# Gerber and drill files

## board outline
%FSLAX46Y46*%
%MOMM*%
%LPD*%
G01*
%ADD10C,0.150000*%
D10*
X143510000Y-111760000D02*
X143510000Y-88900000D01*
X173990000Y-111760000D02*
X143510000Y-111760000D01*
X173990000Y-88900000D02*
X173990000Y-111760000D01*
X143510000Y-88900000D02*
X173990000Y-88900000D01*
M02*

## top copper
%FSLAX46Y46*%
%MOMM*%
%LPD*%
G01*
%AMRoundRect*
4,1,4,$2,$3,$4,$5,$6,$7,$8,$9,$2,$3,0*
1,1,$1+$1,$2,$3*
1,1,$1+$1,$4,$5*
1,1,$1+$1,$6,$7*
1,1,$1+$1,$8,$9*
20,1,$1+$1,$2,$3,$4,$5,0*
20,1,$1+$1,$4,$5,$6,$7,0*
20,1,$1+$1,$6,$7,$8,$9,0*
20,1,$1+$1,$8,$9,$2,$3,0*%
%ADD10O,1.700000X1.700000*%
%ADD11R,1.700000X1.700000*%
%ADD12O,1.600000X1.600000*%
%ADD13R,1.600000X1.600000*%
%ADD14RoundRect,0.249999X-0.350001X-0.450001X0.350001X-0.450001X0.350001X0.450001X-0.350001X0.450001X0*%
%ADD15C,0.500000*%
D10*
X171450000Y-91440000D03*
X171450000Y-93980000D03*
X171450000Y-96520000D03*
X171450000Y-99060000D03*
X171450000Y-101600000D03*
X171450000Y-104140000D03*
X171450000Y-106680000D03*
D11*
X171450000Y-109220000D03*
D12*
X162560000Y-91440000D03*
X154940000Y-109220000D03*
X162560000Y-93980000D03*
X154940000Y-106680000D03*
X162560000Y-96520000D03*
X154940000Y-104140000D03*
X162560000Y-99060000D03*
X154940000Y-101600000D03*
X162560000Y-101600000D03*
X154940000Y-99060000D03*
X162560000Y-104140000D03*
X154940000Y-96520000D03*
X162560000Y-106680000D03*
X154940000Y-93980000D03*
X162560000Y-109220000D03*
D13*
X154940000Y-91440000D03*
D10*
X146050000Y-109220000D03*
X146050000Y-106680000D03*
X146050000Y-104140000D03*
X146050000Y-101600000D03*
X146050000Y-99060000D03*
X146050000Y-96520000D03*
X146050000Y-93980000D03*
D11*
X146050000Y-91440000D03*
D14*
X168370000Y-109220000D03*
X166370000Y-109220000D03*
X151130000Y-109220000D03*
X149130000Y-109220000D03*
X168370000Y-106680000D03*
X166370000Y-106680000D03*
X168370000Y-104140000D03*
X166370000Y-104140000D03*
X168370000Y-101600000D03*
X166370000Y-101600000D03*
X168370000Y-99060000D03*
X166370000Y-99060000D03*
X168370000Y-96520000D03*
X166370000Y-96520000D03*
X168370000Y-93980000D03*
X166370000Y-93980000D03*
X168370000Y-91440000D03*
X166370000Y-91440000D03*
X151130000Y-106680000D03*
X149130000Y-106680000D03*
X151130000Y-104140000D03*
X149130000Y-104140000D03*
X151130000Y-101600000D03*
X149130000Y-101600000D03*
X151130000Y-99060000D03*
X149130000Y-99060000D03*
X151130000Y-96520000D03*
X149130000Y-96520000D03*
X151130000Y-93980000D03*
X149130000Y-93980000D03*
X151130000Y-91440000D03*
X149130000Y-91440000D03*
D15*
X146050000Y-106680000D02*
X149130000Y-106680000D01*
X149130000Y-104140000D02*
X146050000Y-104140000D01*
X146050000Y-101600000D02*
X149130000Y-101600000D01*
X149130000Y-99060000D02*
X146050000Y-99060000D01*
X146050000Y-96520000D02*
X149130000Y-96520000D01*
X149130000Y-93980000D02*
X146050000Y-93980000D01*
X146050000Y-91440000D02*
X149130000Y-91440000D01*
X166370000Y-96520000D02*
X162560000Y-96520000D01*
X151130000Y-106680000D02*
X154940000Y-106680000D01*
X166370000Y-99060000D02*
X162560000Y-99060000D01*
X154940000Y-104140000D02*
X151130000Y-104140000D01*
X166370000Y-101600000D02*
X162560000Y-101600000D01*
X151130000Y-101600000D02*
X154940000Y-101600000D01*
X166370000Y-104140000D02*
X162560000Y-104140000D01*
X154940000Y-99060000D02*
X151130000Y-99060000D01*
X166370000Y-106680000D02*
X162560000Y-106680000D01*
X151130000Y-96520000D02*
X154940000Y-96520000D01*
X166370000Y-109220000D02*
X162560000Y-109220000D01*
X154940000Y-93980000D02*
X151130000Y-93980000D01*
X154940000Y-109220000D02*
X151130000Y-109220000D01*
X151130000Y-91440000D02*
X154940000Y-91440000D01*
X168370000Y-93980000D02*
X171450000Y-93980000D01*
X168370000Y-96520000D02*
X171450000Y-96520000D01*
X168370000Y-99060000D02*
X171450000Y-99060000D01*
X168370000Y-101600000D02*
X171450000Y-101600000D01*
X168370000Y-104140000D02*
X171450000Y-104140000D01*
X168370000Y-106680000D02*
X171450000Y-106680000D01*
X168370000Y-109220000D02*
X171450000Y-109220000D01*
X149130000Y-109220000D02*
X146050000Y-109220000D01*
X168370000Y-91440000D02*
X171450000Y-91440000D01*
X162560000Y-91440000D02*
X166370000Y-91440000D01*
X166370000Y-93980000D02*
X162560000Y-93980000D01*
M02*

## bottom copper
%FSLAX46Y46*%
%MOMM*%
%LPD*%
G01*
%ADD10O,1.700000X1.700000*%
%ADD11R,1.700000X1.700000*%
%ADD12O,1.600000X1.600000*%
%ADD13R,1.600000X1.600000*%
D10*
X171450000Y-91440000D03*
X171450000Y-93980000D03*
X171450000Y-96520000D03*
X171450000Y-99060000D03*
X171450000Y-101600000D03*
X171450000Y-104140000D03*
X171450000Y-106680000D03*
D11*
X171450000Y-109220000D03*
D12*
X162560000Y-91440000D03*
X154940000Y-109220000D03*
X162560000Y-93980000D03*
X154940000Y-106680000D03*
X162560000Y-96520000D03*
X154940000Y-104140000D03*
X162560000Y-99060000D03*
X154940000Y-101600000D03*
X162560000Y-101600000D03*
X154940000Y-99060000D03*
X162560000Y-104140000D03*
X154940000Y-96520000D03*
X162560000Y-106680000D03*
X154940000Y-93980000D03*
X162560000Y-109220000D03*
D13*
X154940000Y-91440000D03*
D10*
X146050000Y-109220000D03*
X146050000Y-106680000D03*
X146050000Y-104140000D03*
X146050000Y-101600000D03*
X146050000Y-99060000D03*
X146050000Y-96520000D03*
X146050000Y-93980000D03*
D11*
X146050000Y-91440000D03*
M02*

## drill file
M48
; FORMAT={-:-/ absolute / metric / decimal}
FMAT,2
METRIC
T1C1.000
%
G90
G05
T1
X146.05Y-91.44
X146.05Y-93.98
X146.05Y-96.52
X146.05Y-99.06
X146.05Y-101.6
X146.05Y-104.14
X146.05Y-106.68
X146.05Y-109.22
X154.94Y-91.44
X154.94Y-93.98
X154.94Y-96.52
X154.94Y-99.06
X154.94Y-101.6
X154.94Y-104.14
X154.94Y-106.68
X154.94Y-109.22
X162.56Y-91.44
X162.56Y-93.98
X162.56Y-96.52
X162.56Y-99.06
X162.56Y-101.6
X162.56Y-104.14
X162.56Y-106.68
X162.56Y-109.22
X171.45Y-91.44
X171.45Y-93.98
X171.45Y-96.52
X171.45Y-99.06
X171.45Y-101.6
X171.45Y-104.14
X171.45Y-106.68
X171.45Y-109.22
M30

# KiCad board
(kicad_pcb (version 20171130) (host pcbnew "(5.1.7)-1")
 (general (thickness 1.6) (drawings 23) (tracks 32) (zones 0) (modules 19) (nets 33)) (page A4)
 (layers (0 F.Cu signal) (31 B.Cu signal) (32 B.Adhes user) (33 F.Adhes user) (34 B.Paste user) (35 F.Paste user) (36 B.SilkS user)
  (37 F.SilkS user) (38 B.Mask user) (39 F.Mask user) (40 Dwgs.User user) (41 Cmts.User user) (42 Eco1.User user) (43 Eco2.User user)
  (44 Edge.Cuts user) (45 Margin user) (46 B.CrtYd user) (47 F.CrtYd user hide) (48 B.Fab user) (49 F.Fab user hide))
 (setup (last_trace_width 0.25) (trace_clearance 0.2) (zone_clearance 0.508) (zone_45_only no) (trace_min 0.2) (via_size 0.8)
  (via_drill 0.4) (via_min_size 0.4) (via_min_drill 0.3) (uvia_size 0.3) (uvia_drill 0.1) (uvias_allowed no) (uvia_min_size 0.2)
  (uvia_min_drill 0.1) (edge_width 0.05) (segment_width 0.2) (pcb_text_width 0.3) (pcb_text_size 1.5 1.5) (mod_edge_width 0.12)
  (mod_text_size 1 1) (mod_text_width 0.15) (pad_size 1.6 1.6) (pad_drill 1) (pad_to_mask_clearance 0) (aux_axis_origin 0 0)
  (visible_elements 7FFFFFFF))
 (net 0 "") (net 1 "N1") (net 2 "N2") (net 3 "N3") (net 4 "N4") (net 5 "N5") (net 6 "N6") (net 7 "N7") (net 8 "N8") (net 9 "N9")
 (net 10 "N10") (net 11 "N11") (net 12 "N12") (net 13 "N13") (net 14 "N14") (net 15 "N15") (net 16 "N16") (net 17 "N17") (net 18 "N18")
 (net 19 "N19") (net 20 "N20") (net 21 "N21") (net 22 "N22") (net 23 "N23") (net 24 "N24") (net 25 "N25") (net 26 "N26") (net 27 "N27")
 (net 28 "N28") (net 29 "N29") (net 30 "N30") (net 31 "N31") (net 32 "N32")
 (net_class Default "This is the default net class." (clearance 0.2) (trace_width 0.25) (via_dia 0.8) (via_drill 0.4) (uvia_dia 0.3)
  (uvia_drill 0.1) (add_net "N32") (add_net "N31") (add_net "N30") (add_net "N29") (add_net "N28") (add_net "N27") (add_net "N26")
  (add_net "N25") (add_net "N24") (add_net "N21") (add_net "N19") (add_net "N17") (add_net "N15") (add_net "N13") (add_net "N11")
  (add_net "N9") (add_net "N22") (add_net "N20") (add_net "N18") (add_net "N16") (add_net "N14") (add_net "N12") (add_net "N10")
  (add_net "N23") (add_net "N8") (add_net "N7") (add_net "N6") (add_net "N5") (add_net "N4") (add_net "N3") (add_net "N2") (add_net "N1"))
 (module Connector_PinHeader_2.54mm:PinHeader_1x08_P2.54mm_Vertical (layer F.Cu) (at 171.45 109.22 180)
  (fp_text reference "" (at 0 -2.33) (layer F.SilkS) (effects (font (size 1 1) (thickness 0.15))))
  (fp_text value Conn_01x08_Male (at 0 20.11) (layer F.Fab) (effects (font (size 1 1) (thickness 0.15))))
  (pad 8 thru_hole oval (at 0 17.78 180) (size 1.7 1.7) (drill 1) (layers *.Cu *.Mask) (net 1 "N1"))
  (pad 7 thru_hole oval (at 0 15.24 180) (size 1.7 1.7) (drill 1) (layers *.Cu *.Mask) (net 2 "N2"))
  (pad 6 thru_hole oval (at 0 12.7 180) (size 1.7 1.7) (drill 1) (layers *.Cu *.Mask) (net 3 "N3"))
  (pad 5 thru_hole oval (at 0 10.16 180) (size 1.7 1.7) (drill 1) (layers *.Cu *.Mask) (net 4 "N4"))
  (pad 4 thru_hole oval (at 0 7.62 180) (size 1.7 1.7) (drill 1) (layers *.Cu *.Mask) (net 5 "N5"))
  (pad 3 thru_hole oval (at 0 5.08 180) (size 1.7 1.7) (drill 1) (layers *.Cu *.Mask) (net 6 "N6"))
  (pad 2 thru_hole oval (at 0 2.54 180) (size 1.7 1.7) (drill 1) (layers *.Cu *.Mask) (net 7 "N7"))
  (pad 1 thru_hole rect (at 0 0 180) (size 1.7 1.7) (drill 1) (layers *.Cu *.Mask) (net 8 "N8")))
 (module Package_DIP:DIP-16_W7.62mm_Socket (layer F.Cu) (at 154.94 91.44)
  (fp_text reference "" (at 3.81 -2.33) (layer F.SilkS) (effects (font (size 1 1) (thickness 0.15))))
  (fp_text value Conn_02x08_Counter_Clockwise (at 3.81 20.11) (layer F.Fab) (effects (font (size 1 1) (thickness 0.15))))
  (pad 16 thru_hole oval (at 7.62 0) (size 1.6 1.6) (drill 1) (layers *.Cu *.Mask) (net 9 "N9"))
  (pad 8 thru_hole oval (at 0 17.78) (size 1.6 1.6) (drill 1) (layers *.Cu *.Mask) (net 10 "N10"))
  (pad 15 thru_hole oval (at 7.62 2.54) (size 1.6 1.6) (drill 1) (layers *.Cu *.Mask) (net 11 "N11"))
  (pad 7 thru_hole oval (at 0 15.24) (size 1.6 1.6) (drill 1) (layers *.Cu *.Mask) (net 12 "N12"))
  (pad 14 thru_hole oval (at 7.62 5.08) (size 1.6 1.6) (drill 1) (layers *.Cu *.Mask) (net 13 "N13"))
  (pad 6 thru_hole oval (at 0 12.7) (size 1.6 1.6) (drill 1) (layers *.Cu *.Mask) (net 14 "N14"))
  (pad 13 thru_hole oval (at 7.62 7.62) (size 1.6 1.6) (drill 1) (layers *.Cu *.Mask) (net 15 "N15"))
  (pad 5 thru_hole oval (at 0 10.16) (size 1.6 1.6) (drill 1) (layers *.Cu *.Mask) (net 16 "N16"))
  (pad 12 thru_hole oval (at 7.62 10.16) (size 1.6 1.6) (drill 1) (layers *.Cu *.Mask) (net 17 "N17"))
  (pad 4 thru_hole oval (at 0 7.62) (size 1.6 1.6) (drill 1) (layers *.Cu *.Mask) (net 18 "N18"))
  (pad 11 thru_hole oval (at 7.62 12.7) (size 1.6 1.6) (drill 1) (layers *.Cu *.Mask) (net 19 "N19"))
  (pad 3 thru_hole oval (at 0 5.08) (size 1.6 1.6) (drill 1) (layers *.Cu *.Mask) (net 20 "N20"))
  (pad 10 thru_hole oval (at 7.62 15.24) (size 1.6 1.6) (drill 1) (layers *.Cu *.Mask) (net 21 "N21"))
  (pad 2 thru_hole oval (at 0 2.54) (size 1.6 1.6) (drill 1) (layers *.Cu *.Mask) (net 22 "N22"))
  (pad 9 thru_hole oval (at 7.62 17.78) (size 1.6 1.6) (drill 1) (layers *.Cu *.Mask) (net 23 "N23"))
  (pad 1 thru_hole rect (at 0 0) (size 1.6 1.6) (drill 1) (layers *.Cu *.Mask) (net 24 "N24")))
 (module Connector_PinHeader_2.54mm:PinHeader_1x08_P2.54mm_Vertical (layer F.Cu) (at 146.05 91.44)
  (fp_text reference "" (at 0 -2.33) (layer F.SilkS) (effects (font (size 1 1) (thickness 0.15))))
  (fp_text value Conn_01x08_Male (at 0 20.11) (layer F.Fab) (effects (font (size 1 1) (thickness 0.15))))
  (pad 8 thru_hole oval (at 0 17.78) (size 1.7 1.7) (drill 1) (layers *.Cu *.Mask) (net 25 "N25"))
  (pad 7 thru_hole oval (at 0 15.24) (size 1.7 1.7) (drill 1) (layers *.Cu *.Mask) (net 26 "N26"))
  (pad 6 thru_hole oval (at 0 12.7) (size 1.7 1.7) (drill 1) (layers *.Cu *.Mask) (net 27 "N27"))
  (pad 5 thru_hole oval (at 0 10.16) (size 1.7 1.7) (drill 1) (layers *.Cu *.Mask) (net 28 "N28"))
  (pad 4 thru_hole oval (at 0 7.62) (size 1.7 1.7) (drill 1) (layers *.Cu *.Mask) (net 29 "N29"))
  (pad 3 thru_hole oval (at 0 5.08) (size 1.7 1.7) (drill 1) (layers *.Cu *.Mask) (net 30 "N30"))
  (pad 2 thru_hole oval (at 0 2.54) (size 1.7 1.7) (drill 1) (layers *.Cu *.Mask) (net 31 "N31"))
  (pad 1 thru_hole rect (at 0 0) (size 1.7 1.7) (drill 1) (layers *.Cu *.Mask) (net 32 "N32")))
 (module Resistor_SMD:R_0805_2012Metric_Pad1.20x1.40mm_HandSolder (layer F.Cu) (at 167.37 109.22)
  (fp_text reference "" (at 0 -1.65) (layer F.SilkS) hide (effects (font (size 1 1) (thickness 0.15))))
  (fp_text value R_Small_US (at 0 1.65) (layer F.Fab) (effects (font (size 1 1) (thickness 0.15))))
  (pad 2 smd roundrect (at 1 0) (size 1.2 1.4) (layers F.Cu F.Paste F.Mask) (roundrect_rratio 0.2083325) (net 8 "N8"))
  (pad 1 smd roundrect (at -1 0) (size 1.2 1.4) (layers F.Cu F.Paste F.Mask) (roundrect_rratio 0.2083325) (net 23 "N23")))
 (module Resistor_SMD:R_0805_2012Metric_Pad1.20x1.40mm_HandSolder (layer F.Cu) (at 150.13 109.22)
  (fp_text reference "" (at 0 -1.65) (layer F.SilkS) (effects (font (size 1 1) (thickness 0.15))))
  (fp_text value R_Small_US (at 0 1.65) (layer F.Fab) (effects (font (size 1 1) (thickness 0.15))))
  (pad 2 smd roundrect (at 1 0) (size 1.2 1.4) (layers F.Cu F.Paste F.Mask) (roundrect_rratio 0.2083325) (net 10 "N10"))
  (pad 1 smd roundrect (at -1 0) (size 1.2 1.4) (layers F.Cu F.Paste F.Mask) (roundrect_rratio 0.2083325) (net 25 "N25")))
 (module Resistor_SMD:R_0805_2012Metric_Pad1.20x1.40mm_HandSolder (layer F.Cu) (at 167.37 106.68)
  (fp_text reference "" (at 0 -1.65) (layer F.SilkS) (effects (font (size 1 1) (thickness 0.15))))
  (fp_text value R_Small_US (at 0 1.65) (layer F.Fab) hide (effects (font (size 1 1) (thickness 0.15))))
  (pad 2 smd roundrect (at 1 0) (size 1.2 1.4) (layers F.Cu F.Paste F.Mask) (roundrect_rratio 0.2083325) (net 7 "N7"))
  (pad 1 smd roundrect (at -1 0) (size 1.2 1.4) (layers F.Cu F.Paste F.Mask) (roundrect_rratio 0.2083325) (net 21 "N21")))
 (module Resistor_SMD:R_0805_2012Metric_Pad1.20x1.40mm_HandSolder (layer F.Cu) (at 167.37 104.14)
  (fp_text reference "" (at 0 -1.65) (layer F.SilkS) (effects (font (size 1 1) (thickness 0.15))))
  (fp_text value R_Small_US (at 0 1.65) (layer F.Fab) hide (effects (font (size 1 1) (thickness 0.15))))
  (pad 2 smd roundrect (at 1 0) (size 1.2 1.4) (layers F.Cu F.Paste F.Mask) (roundrect_rratio 0.2083325) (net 6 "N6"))
  (pad 1 smd roundrect (at -1 0) (size 1.2 1.4) (layers F.Cu F.Paste F.Mask) (roundrect_rratio 0.2083325) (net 19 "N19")))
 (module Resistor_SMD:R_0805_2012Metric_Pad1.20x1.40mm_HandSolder (layer F.Cu) (at 167.37 101.6)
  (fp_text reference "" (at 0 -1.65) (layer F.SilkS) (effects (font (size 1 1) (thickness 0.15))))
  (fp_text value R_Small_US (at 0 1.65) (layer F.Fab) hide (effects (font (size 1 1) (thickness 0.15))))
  (pad 2 smd roundrect (at 1 0) (size 1.2 1.4) (layers F.Cu F.Paste F.Mask) (roundrect_rratio 0.2083325) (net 5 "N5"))
  (pad 1 smd roundrect (at -1 0) (size 1.2 1.4) (layers F.Cu F.Paste F.Mask) (roundrect_rratio 0.2083325) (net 17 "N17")))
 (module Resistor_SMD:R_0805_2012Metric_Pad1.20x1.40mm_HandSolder (layer F.Cu) (at 167.37 99.06)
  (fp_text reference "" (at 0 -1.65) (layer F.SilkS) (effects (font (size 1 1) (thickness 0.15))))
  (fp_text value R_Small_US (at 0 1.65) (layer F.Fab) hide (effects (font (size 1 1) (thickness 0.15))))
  (pad 2 smd roundrect (at 1 0) (size 1.2 1.4) (layers F.Cu F.Paste F.Mask) (roundrect_rratio 0.2083325) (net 4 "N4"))
  (pad 1 smd roundrect (at -1 0) (size 1.2 1.4) (layers F.Cu F.Paste F.Mask) (roundrect_rratio 0.2083325) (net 15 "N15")))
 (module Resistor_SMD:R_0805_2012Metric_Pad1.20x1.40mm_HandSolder (layer F.Cu) (at 167.37 96.52)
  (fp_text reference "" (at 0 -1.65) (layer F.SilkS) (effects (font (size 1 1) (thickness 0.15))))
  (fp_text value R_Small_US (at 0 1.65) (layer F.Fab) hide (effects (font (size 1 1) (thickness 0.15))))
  (pad 2 smd roundrect (at 1 0) (size 1.2 1.4) (layers F.Cu F.Paste F.Mask) (roundrect_rratio 0.2083325) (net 3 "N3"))
  (pad 1 smd roundrect (at -1 0) (size 1.2 1.4) (layers F.Cu F.Paste F.Mask) (roundrect_rratio 0.2083325) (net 13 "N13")))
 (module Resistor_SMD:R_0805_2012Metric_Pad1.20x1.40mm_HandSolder (layer F.Cu) (at 167.37 93.98)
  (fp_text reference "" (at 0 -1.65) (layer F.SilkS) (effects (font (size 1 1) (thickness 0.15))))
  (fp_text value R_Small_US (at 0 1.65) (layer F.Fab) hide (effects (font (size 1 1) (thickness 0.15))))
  (pad 2 smd roundrect (at 1 0) (size 1.2 1.4) (layers F.Cu F.Paste F.Mask) (roundrect_rratio 0.2083325) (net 2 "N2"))
  (pad 1 smd roundrect (at -1 0) (size 1.2 1.4) (layers F.Cu F.Paste F.Mask) (roundrect_rratio 0.2083325) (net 11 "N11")))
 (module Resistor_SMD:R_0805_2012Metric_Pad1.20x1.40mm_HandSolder (layer F.Cu) (at 167.37 91.44)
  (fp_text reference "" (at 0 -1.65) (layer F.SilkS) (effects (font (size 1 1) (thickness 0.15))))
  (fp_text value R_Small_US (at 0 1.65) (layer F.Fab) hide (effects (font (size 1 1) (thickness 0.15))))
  (pad 2 smd roundrect (at 1 0) (size 1.2 1.4) (layers F.Cu F.Paste F.Mask) (roundrect_rratio 0.2083325) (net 1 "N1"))
  (pad 1 smd roundrect (at -1 0) (size 1.2 1.4) (layers F.Cu F.Paste F.Mask) (roundrect_rratio 0.2083325) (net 9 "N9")))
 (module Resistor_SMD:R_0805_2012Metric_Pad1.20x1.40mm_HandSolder (layer F.Cu) (at 150.13 106.68)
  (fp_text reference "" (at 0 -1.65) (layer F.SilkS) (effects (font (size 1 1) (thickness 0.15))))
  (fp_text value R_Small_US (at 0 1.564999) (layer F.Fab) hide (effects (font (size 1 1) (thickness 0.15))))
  (pad 2 smd roundrect (at 1 0) (size 1.2 1.4) (layers F.Cu F.Paste F.Mask) (roundrect_rratio 0.2083325) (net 12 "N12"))
  (pad 1 smd roundrect (at -1 0) (size 1.2 1.4) (layers F.Cu F.Paste F.Mask) (roundrect_rratio 0.2083325) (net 26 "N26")))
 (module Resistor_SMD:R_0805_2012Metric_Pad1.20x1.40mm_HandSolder (layer F.Cu) (at 150.13 104.14)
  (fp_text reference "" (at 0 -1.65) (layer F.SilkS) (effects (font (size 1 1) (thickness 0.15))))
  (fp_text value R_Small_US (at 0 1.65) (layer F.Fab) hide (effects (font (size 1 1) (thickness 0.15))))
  (pad 2 smd roundrect (at 1 0) (size 1.2 1.4) (layers F.Cu F.Paste F.Mask) (roundrect_rratio 0.2083325) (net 14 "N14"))
  (pad 1 smd roundrect (at -1 0) (size 1.2 1.4) (layers F.Cu F.Paste F.Mask) (roundrect_rratio 0.2083325) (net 27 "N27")))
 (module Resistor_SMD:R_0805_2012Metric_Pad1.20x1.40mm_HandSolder (layer F.Cu) (at 150.13 101.6)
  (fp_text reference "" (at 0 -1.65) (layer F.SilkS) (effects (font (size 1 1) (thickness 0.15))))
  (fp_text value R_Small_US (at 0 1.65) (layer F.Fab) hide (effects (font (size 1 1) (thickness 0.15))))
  (pad 2 smd roundrect (at 1 0) (size 1.2 1.4) (layers F.Cu F.Paste F.Mask) (roundrect_rratio 0.2083325) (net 16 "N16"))
  (pad 1 smd roundrect (at -1 0) (size 1.2 1.4) (layers F.Cu F.Paste F.Mask) (roundrect_rratio 0.2083325) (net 28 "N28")))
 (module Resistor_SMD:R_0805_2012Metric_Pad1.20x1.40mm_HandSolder (layer F.Cu) (at 150.13 99.06)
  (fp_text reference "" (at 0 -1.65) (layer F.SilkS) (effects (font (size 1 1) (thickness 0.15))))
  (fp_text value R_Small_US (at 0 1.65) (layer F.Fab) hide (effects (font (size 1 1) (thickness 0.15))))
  (pad 2 smd roundrect (at 1 0) (size 1.2 1.4) (layers F.Cu F.Paste F.Mask) (roundrect_rratio 0.2083325) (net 18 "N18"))
  (pad 1 smd roundrect (at -1 0) (size 1.2 1.4) (layers F.Cu F.Paste F.Mask) (roundrect_rratio 0.2083325) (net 29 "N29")))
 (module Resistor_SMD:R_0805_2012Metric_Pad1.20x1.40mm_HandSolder (layer F.Cu) (at 150.13 96.52)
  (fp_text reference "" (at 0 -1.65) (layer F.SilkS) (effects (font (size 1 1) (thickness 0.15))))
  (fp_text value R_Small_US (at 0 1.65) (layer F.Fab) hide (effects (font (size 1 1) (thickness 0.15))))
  (pad 2 smd roundrect (at 1 0) (size 1.2 1.4) (layers F.Cu F.Paste F.Mask) (roundrect_rratio 0.2083325) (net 20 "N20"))
  (pad 1 smd roundrect (at -1 0) (size 1.2 1.4) (layers F.Cu F.Paste F.Mask) (roundrect_rratio 0.2083325) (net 30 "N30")))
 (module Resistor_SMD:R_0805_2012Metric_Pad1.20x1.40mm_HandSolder (layer F.Cu) (at 150.13 93.98)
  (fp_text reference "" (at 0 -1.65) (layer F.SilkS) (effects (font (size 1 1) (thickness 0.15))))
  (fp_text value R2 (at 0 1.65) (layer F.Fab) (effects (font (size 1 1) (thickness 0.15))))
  (pad 2 smd roundrect (at 1 0) (size 1.2 1.4) (layers F.Cu F.Paste F.Mask) (roundrect_rratio 0.2083325) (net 22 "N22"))
  (pad 1 smd roundrect (at -1 0) (size 1.2 1.4) (layers F.Cu F.Paste F.Mask) (roundrect_rratio 0.2083325) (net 31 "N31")))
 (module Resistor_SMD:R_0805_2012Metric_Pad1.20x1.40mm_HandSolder (layer F.Cu) (at 150.13 91.44)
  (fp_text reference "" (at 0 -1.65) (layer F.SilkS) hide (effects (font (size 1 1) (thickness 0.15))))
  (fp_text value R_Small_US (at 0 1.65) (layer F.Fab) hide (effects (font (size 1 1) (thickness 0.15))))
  (pad 2 smd roundrect (at 1 0) (size 1.2 1.4) (layers F.Cu F.Paste F.Mask) (roundrect_rratio 0.2083325) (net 24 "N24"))
  (pad 1 smd roundrect (at -1 0) (size 1.2 1.4) (layers F.Cu F.Paste F.Mask) (roundrect_rratio 0.2083325) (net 32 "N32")))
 (gr_line (start 143.51 111.76) (end 143.51 88.9) (layer Edge.Cuts) (width 0.15))
 (gr_line (start 173.99 111.76) (end 143.51 111.76) (layer Edge.Cuts) (width 0.15))
 (gr_line (start 173.99 88.9) (end 173.99 111.76) (layer Edge.Cuts) (width 0.15))
 (gr_line (start 143.51 88.9) (end 173.99 88.9) (layer Edge.Cuts) (width 0.15))
 (segment (start 146.05 106.68) (end 149.13 106.68) (width 0.5) (layer F.Cu) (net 26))
 (segment (start 149.13 104.14) (end 146.05 104.14) (width 0.5) (layer F.Cu) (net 27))
 (segment (start 146.05 101.6) (end 149.13 101.6) (width 0.5) (layer F.Cu) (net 28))
 (segment (start 149.13 99.06) (end 146.05 99.06) (width 0.5) (layer F.Cu) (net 29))
 (segment (start 146.05 96.52) (end 149.13 96.52) (width 0.5) (layer F.Cu) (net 30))
 (segment (start 149.13 93.98) (end 146.05 93.98) (width 0.5) (layer F.Cu) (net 31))
 (segment (start 146.05 91.44) (end 149.13 91.44) (width 0.5) (layer F.Cu) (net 32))
 (segment (start 166.37 96.52) (end 162.56 96.52) (width 0.5) (layer F.Cu) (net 13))
 (segment (start 151.13 106.68) (end 154.94 106.68) (width 0.5) (layer F.Cu) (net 12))
 (segment (start 166.37 99.06) (end 162.56 99.06) (width 0.5) (layer F.Cu) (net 15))
 (segment (start 154.94 104.14) (end 151.13 104.14) (width 0.5) (layer F.Cu) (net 14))
 (segment (start 166.37 101.6) (end 162.56 101.6) (width 0.5) (layer F.Cu) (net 17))
 (segment (start 151.13 101.6) (end 154.94 101.6) (width 0.5) (layer F.Cu) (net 16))
 (segment (start 166.37 104.14) (end 162.56 104.14) (width 0.5) (layer F.Cu) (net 19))
 (segment (start 154.94 99.06) (end 151.13 99.06) (width 0.5) (layer F.Cu) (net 18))
 (segment (start 166.37 106.68) (end 162.56 106.68) (width 0.5) (layer F.Cu) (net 21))
 (segment (start 151.13 96.52) (end 154.94 96.52) (width 0.5) (layer F.Cu) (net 20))
 (segment (start 166.37 109.22) (end 162.56 109.22) (width 0.5) (layer F.Cu) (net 23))
 (segment (start 154.94 93.98) (end 151.13 93.98) (width 0.5) (layer F.Cu) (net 22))
 (segment (start 154.94 109.22) (end 151.13 109.22) (width 0.5) (layer F.Cu) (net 10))
 (segment (start 151.13 91.44) (end 154.94 91.44) (width 0.5) (layer F.Cu) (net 24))
 (segment (start 168.37 93.98) (end 171.45 93.98) (width 0.5) (layer F.Cu) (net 2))
 (segment (start 168.37 96.52) (end 171.45 96.52) (width 0.5) (layer F.Cu) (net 3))
 (segment (start 168.37 99.06) (end 171.45 99.06) (width 0.5) (layer F.Cu) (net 4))
 (segment (start 168.37 101.6) (end 171.45 101.6) (width 0.5) (layer F.Cu) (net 5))
 (segment (start 168.37 104.14) (end 171.45 104.14) (width 0.5) (layer F.Cu) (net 6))
 (segment (start 168.37 106.68) (end 171.45 106.68) (width 0.5) (layer F.Cu) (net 7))
 (segment (start 168.37 109.22) (end 171.45 109.22) (width 0.5) (layer F.Cu) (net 8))
 (segment (start 149.13 109.22) (end 146.05 109.22) (width 0.5) (layer F.Cu) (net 25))
 (segment (start 168.37 91.44) (end 171.45 91.44) (width 0.5) (layer F.Cu) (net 1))
 (segment (start 162.56 91.44) (end 166.37 91.44) (width 0.5) (layer F.Cu) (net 9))
 (segment (start 166.37 93.98) (end 162.56 93.98) (width 0.5) (layer F.Cu) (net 11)))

